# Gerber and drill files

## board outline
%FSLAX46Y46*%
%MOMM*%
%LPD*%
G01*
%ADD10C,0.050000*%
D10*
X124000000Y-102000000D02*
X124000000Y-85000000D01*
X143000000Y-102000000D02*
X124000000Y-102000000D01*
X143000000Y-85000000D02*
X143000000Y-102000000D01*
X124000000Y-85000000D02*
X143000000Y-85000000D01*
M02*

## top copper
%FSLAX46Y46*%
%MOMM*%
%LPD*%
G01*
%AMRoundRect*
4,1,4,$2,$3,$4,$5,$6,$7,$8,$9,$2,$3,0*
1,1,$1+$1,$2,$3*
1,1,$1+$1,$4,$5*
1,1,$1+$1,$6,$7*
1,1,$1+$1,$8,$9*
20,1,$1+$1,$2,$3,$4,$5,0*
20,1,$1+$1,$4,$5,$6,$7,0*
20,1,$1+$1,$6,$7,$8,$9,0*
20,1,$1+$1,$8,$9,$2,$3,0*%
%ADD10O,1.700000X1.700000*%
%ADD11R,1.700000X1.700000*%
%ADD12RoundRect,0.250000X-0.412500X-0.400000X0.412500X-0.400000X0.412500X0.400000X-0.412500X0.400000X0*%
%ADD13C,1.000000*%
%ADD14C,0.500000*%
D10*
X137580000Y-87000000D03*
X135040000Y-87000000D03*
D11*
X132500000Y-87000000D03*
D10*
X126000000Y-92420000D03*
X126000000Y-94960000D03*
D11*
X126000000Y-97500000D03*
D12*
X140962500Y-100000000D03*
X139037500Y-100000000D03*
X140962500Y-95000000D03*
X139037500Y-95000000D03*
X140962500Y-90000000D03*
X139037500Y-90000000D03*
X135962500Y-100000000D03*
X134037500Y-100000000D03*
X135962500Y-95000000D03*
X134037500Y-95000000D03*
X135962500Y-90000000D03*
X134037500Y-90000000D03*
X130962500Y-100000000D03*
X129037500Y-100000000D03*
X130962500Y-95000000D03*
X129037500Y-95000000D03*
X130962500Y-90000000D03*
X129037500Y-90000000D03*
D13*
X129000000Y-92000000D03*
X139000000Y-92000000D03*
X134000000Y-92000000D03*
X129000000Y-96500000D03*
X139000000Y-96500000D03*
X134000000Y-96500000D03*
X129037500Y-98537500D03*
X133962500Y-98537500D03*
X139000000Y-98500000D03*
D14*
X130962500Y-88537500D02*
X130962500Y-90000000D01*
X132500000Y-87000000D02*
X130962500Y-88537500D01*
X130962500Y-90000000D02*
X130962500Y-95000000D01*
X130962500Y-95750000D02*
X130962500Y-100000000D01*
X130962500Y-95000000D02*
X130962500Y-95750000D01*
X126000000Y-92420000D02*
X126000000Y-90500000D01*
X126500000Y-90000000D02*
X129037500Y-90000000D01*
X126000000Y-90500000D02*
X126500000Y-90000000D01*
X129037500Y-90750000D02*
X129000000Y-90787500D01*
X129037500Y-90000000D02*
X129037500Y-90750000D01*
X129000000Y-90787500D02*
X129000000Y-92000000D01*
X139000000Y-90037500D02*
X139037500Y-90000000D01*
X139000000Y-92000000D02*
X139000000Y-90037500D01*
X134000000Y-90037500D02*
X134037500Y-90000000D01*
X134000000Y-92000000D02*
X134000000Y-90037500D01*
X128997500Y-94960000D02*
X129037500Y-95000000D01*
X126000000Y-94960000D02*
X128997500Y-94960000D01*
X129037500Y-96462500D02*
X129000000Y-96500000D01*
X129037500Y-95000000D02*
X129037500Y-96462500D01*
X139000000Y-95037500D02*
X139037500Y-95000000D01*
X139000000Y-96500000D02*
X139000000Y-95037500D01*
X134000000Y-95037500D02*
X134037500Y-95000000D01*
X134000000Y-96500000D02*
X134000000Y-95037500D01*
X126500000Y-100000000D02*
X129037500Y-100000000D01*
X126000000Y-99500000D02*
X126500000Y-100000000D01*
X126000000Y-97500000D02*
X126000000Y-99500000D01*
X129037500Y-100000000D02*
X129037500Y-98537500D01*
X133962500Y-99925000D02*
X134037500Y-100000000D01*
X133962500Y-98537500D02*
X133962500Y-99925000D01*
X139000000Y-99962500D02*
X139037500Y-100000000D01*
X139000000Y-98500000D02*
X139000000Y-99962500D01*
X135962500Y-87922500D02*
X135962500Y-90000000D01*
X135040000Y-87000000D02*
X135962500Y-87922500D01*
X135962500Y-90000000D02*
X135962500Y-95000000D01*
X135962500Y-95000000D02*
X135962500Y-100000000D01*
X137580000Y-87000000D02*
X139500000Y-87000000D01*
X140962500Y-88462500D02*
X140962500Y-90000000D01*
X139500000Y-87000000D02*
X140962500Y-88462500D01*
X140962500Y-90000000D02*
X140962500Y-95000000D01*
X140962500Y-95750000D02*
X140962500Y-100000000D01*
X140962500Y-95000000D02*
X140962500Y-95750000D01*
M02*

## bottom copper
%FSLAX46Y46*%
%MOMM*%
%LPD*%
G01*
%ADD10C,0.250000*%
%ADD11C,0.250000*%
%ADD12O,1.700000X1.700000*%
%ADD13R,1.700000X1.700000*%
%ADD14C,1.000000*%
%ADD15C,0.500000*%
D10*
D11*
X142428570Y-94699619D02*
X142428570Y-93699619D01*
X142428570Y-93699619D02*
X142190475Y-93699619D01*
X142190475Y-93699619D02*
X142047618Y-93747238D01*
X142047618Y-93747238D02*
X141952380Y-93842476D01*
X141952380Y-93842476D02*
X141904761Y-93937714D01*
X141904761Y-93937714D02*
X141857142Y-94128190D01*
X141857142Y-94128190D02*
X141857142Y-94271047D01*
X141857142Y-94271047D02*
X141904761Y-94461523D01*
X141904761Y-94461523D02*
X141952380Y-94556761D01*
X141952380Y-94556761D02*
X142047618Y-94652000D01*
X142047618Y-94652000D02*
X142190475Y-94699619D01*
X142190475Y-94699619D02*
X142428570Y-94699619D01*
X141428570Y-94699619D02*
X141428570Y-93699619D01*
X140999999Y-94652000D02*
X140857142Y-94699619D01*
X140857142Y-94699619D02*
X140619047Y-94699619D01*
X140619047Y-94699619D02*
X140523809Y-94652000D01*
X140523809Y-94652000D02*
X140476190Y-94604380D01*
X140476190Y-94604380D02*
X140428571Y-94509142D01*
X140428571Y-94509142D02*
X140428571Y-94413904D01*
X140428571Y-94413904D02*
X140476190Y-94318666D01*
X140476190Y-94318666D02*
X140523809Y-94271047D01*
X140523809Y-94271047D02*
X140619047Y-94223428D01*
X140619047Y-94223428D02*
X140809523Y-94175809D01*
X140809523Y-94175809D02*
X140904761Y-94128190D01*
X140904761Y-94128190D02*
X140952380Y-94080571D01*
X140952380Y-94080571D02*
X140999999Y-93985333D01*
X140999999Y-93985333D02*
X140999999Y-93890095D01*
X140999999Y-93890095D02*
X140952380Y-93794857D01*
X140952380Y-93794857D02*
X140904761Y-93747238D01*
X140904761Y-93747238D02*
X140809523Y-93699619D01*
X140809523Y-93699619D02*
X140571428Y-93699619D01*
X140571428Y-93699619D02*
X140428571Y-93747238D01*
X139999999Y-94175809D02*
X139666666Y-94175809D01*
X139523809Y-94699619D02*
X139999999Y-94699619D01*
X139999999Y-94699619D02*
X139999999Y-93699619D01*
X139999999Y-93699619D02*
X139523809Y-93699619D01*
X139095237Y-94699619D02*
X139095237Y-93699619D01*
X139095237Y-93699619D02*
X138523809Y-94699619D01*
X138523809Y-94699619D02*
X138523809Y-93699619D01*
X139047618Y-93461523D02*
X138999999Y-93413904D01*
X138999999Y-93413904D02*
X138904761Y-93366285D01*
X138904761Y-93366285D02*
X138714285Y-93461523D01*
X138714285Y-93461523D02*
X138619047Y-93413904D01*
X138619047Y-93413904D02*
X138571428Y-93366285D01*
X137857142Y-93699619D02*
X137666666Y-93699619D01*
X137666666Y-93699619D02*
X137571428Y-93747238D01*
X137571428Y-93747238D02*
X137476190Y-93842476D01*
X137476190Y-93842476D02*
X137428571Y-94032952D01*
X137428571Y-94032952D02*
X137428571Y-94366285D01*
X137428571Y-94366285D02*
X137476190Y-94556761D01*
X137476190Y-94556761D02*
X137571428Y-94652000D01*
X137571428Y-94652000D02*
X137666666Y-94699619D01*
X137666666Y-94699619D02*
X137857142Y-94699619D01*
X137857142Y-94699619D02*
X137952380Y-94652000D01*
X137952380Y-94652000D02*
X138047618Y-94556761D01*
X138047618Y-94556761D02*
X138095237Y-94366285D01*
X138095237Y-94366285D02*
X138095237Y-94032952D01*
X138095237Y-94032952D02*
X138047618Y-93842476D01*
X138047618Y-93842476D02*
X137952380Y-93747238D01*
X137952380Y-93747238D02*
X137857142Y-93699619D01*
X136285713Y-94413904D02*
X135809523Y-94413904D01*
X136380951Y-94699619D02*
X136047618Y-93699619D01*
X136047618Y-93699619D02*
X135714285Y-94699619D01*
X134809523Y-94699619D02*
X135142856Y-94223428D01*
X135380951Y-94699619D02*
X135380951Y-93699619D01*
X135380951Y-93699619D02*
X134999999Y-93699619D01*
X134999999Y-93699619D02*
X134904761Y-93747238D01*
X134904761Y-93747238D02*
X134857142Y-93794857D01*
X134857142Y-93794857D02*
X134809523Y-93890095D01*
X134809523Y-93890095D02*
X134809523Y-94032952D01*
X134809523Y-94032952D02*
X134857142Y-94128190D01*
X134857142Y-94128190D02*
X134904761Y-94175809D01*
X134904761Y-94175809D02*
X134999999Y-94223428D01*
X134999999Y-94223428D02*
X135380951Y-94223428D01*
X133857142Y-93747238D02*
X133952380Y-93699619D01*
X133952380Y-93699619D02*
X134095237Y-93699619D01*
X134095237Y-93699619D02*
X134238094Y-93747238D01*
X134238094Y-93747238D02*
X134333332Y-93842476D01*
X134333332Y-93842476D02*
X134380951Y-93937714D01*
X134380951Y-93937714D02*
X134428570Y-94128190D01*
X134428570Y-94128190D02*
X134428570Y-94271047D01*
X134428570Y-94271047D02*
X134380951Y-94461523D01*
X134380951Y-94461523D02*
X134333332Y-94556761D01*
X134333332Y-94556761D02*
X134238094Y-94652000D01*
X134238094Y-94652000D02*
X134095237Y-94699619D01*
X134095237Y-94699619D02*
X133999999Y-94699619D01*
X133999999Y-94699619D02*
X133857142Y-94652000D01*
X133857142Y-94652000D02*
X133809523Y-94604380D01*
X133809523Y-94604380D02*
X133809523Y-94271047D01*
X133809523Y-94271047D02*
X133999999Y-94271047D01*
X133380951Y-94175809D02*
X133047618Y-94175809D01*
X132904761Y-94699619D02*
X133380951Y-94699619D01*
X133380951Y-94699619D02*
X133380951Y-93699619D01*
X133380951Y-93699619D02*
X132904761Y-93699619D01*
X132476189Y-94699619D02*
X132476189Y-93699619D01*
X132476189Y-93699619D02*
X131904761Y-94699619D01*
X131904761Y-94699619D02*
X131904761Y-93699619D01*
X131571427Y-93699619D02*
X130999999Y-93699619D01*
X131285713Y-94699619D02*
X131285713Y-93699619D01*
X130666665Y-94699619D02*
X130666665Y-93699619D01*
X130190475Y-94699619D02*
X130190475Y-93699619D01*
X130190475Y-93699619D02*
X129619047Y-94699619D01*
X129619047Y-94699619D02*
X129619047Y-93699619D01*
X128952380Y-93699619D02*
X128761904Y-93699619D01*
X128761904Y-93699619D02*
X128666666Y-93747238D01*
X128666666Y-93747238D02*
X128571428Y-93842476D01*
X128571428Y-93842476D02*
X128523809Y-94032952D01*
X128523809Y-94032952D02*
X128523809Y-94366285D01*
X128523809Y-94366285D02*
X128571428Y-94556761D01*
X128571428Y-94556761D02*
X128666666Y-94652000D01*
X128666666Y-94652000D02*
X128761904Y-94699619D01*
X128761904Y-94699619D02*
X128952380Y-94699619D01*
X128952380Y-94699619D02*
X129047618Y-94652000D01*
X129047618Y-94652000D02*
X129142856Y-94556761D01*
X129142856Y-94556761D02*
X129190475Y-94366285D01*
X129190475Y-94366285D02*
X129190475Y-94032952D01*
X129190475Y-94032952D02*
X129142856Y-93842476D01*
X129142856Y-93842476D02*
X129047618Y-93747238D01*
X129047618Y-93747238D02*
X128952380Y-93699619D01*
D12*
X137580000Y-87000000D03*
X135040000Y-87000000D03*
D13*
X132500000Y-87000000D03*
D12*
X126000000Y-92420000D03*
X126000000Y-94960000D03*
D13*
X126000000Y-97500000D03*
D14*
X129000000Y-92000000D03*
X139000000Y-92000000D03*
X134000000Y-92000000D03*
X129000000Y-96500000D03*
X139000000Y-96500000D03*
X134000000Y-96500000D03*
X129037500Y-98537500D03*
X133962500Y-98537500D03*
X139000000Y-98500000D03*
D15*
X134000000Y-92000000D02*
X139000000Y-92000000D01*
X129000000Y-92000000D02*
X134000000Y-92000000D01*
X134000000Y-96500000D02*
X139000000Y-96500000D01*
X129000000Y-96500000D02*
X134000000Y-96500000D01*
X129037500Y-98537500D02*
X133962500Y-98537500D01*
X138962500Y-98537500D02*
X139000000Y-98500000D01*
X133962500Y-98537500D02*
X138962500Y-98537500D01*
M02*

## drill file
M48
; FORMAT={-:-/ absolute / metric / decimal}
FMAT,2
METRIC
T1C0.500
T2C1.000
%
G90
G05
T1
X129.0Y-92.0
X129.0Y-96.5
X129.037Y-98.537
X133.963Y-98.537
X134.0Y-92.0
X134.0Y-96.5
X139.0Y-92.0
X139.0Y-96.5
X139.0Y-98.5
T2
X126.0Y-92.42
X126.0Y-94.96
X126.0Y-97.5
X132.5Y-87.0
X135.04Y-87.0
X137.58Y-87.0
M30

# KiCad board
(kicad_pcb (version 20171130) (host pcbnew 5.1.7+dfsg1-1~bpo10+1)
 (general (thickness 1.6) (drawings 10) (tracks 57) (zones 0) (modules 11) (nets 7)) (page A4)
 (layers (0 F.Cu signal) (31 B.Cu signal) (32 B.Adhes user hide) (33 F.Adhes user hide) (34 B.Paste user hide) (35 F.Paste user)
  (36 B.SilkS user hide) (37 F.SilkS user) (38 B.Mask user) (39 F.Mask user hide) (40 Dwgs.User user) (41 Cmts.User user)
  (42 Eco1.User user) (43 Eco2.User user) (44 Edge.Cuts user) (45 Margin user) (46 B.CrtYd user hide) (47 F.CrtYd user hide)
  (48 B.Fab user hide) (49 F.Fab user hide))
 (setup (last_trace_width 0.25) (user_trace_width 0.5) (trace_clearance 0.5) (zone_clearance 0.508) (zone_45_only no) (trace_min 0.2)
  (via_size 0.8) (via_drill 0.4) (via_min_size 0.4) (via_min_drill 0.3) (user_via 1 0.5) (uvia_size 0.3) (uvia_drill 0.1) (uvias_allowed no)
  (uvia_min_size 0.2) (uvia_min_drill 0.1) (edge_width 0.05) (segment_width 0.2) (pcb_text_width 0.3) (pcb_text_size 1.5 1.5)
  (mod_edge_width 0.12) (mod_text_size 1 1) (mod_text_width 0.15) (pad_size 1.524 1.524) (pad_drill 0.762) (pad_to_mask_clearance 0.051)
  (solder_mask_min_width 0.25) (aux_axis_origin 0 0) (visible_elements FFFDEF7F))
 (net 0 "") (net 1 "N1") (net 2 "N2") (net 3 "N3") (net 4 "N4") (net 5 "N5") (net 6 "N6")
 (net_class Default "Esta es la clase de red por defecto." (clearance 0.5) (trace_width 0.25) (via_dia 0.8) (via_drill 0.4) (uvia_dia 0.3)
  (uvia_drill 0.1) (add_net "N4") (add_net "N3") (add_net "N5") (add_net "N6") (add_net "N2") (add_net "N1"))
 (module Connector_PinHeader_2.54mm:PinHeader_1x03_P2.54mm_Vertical (layer B.Cu) (at 132.5 87 270)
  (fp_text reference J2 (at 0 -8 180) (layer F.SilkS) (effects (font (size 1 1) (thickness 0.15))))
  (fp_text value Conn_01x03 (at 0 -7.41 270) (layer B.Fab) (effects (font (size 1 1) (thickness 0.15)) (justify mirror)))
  (pad 3 thru_hole oval (at 0 -5.08 270) (size 1.7 1.7) (drill 1) (layers *.Cu *.Mask) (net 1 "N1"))
  (pad 2 thru_hole oval (at 0 -2.54 270) (size 1.7 1.7) (drill 1) (layers *.Cu *.Mask) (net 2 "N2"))
  (pad 1 thru_hole rect (at 0 0 270) (size 1.7 1.7) (drill 1) (layers *.Cu *.Mask) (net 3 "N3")))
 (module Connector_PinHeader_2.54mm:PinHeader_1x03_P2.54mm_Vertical (layer B.Cu) (at 126 97.5)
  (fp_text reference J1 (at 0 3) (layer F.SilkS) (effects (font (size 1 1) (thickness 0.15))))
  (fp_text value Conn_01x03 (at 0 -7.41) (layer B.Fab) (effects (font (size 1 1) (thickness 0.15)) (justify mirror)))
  (pad 3 thru_hole oval (at 0 -5.08) (size 1.7 1.7) (drill 1) (layers *.Cu *.Mask) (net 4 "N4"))
  (pad 2 thru_hole oval (at 0 -2.54) (size 1.7 1.7) (drill 1) (layers *.Cu *.Mask) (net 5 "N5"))
  (pad 1 thru_hole rect (at 0 0) (size 1.7 1.7) (drill 1) (layers *.Cu *.Mask) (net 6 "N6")))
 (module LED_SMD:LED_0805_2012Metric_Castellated (layer F.Cu) (at 140 100)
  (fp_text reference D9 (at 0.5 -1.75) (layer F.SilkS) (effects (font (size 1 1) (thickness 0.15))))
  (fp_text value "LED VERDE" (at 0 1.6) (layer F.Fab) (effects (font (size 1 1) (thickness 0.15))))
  (pad 2 smd roundrect (at 0.9625 0) (size 1.325 1.3) (layers F.Cu F.Paste F.Mask) (roundrect_rratio 0.192308) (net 1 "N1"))
  (pad 1 smd roundrect (at -0.9625 0) (size 1.325 1.3) (layers F.Cu F.Paste F.Mask) (roundrect_rratio 0.192308) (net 6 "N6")))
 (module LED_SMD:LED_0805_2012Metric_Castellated (layer F.Cu) (at 140 95)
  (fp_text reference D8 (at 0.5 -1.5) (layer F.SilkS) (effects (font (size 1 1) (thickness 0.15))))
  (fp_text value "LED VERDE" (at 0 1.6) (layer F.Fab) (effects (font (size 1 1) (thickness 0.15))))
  (pad 2 smd roundrect (at 0.9625 0) (size 1.325 1.3) (layers F.Cu F.Paste F.Mask) (roundrect_rratio 0.192308) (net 1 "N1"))
  (pad 1 smd roundrect (at -0.9625 0) (size 1.325 1.3) (layers F.Cu F.Paste F.Mask) (roundrect_rratio 0.192308) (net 5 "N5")))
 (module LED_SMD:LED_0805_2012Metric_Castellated (layer F.Cu) (at 140 90)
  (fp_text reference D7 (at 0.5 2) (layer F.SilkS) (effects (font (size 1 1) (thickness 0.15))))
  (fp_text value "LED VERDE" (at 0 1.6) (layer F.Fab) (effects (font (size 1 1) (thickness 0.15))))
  (pad 2 smd roundrect (at 0.9625 0) (size 1.325 1.3) (layers F.Cu F.Paste F.Mask) (roundrect_rratio 0.192308) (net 1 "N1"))
  (pad 1 smd roundrect (at -0.9625 0) (size 1.325 1.3) (layers F.Cu F.Paste F.Mask) (roundrect_rratio 0.192308) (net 4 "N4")))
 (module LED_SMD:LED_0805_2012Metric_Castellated (layer F.Cu) (at 135 100)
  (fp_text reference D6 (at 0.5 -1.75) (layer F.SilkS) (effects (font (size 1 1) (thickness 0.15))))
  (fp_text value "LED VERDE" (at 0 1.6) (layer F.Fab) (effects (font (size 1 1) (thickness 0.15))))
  (pad 2 smd roundrect (at 0.9625 0) (size 1.325 1.3) (layers F.Cu F.Paste F.Mask) (roundrect_rratio 0.192308) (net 2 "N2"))
  (pad 1 smd roundrect (at -0.9625 0) (size 1.325 1.3) (layers F.Cu F.Paste F.Mask) (roundrect_rratio 0.192308) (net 6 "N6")))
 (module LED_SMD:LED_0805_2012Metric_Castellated (layer F.Cu) (at 135 95)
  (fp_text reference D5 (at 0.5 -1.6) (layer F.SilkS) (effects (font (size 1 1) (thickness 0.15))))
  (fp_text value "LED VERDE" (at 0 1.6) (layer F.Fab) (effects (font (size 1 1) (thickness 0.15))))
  (pad 2 smd roundrect (at 0.9625 0) (size 1.325 1.3) (layers F.Cu F.Paste F.Mask) (roundrect_rratio 0.192308) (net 2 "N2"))
  (pad 1 smd roundrect (at -0.9625 0) (size 1.325 1.3) (layers F.Cu F.Paste F.Mask) (roundrect_rratio 0.192308) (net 5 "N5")))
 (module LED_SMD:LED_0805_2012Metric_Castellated (layer F.Cu) (at 135 90)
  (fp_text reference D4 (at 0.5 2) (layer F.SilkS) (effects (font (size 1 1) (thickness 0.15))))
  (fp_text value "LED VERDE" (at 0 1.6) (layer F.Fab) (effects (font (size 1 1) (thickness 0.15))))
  (pad 2 smd roundrect (at 0.9625 0) (size 1.325 1.3) (layers F.Cu F.Paste F.Mask) (roundrect_rratio 0.192308) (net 2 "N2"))
  (pad 1 smd roundrect (at -0.9625 0) (size 1.325 1.3) (layers F.Cu F.Paste F.Mask) (roundrect_rratio 0.192308) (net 4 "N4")))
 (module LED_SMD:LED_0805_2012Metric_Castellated (layer F.Cu) (at 130 100)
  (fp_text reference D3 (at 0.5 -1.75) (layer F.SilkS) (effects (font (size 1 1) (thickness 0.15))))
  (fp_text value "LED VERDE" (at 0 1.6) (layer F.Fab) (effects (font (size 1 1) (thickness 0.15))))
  (pad 2 smd roundrect (at 0.9625 0) (size 1.325 1.3) (layers F.Cu F.Paste F.Mask) (roundrect_rratio 0.192308) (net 3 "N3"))
  (pad 1 smd roundrect (at -0.9625 0) (size 1.325 1.3) (layers F.Cu F.Paste F.Mask) (roundrect_rratio 0.192308) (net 6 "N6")))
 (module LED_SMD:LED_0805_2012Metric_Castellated (layer F.Cu) (at 130 95)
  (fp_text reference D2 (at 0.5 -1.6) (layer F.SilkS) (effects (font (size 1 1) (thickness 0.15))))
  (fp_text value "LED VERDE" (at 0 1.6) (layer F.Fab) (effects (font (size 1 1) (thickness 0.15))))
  (pad 2 smd roundrect (at 0.9625 0) (size 1.325 1.3) (layers F.Cu F.Paste F.Mask) (roundrect_rratio 0.192308) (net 3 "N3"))
  (pad 1 smd roundrect (at -0.9625 0) (size 1.325 1.3) (layers F.Cu F.Paste F.Mask) (roundrect_rratio 0.192308) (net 5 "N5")))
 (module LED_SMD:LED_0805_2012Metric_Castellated (layer F.Cu) (at 130 90)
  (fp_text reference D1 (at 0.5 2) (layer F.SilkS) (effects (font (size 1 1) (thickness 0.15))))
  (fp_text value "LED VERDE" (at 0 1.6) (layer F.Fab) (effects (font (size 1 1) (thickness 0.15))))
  (pad 2 smd roundrect (at 0.9625 0) (size 1.325 1.3) (layers F.Cu F.Paste F.Mask) (roundrect_rratio 0.192308) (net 3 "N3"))
  (pad 1 smd roundrect (at -0.9625 0) (size 1.325 1.3) (layers F.Cu F.Paste F.Mask) (roundrect_rratio 0.192308) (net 4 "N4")))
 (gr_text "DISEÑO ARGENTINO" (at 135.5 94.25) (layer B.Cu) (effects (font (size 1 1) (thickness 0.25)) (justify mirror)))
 (gr_line (start 124 102) (end 124 85) (layer Edge.Cuts) (width 0.05))
 (gr_line (start 143 102) (end 124 102) (layer Edge.Cuts) (width 0.05))
 (gr_line (start 143 85) (end 143 102) (layer Edge.Cuts) (width 0.05))
 (gr_line (start 124 85) (end 143 85) (layer Edge.Cuts) (width 0.05))
 (segment (start 130.9625 88.5375) (end 130.9625 90) (width 0.5) (layer F.Cu) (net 3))
 (segment (start 132.5 87) (end 130.9625 88.5375) (width 0.5) (layer F.Cu) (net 3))
 (segment (start 130.9625 90) (end 130.9625 95) (width 0.5) (layer F.Cu) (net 3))
 (segment (start 130.9625 95.75) (end 130.9625 100) (width 0.5) (layer F.Cu) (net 3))
 (segment (start 130.9625 95) (end 130.9625 95.75) (width 0.5) (layer F.Cu) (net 3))
 (segment (start 126 92.42) (end 126 90.5) (width 0.5) (layer F.Cu) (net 4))
 (segment (start 126.5 90) (end 129.0375 90) (width 0.5) (layer F.Cu) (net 4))
 (segment (start 126 90.5) (end 126.5 90) (width 0.5) (layer F.Cu) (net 4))
 (segment (start 129.0375 90.75) (end 129 90.7875) (width 0.5) (layer F.Cu) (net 4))
 (segment (start 129.0375 90) (end 129.0375 90.75) (width 0.5) (layer F.Cu) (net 4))
 (via (at 129 92) (size 1) (drill 0.5) (layers F.Cu B.Cu) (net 4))
 (segment (start 129 90.7875) (end 129 92) (width 0.5) (layer F.Cu) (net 4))
 (via (at 139 92) (size 1) (drill 0.5) (layers F.Cu B.Cu) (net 4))
 (segment (start 139 90.0375) (end 139.0375 90) (width 0.5) (layer F.Cu) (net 4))
 (segment (start 139 92) (end 139 90.0375) (width 0.5) (layer F.Cu) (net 4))
 (segment (start 134 92) (end 139 92) (width 0.5) (layer B.Cu) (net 4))
 (segment (start 129 92) (end 134 92) (width 0.5) (layer B.Cu) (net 4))
 (via (at 134 92) (size 1) (drill 0.5) (layers F.Cu B.Cu) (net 4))
 (segment (start 134 90.0375) (end 134.0375 90) (width 0.5) (layer F.Cu) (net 4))
 (segment (start 134 92) (end 134 90.0375) (width 0.5) (layer F.Cu) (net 4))
 (segment (start 128.9975 94.96) (end 129.0375 95) (width 0.5) (layer F.Cu) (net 5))
 (segment (start 126 94.96) (end 128.9975 94.96) (width 0.5) (layer F.Cu) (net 5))
 (via (at 129 96.5) (size 1) (drill 0.5) (layers F.Cu B.Cu) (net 5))
 (segment (start 129.0375 96.4625) (end 129 96.5) (width 0.5) (layer F.Cu) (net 5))
 (segment (start 129.0375 95) (end 129.0375 96.4625) (width 0.5) (layer F.Cu) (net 5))
 (via (at 139 96.5) (size 1) (drill 0.5) (layers F.Cu B.Cu) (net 5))
 (segment (start 139 95.0375) (end 139.0375 95) (width 0.5) (layer F.Cu) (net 5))
 (segment (start 139 96.5) (end 139 95.0375) (width 0.5) (layer F.Cu) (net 5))
 (segment (start 134 96.5) (end 139 96.5) (width 0.5) (layer B.Cu) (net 5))
 (segment (start 129 96.5) (end 134 96.5) (width 0.5) (layer B.Cu) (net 5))
 (via (at 134 96.5) (size 1) (drill 0.5) (layers F.Cu B.Cu) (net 5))
 (segment (start 134 95.0375) (end 134.0375 95) (width 0.5) (layer F.Cu) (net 5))
 (segment (start 134 96.5) (end 134 95.0375) (width 0.5) (layer F.Cu) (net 5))
 (segment (start 126.5 100) (end 129.0375 100) (width 0.5) (layer F.Cu) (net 6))
 (segment (start 126 99.5) (end 126.5 100) (width 0.5) (layer F.Cu) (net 6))
 (segment (start 126 97.5) (end 126 99.5) (width 0.5) (layer F.Cu) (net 6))
 (segment (start 129.0375 100) (end 129.0375 98.5375) (width 0.5) (layer F.Cu) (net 6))
 (via (at 129.0375 98.5375) (size 1) (drill 0.5) (layers F.Cu B.Cu) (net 6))
 (segment (start 129.0375 98.5375) (end 133.9625 98.5375) (width 0.5) (layer B.Cu) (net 6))
 (via (at 133.9625 98.5375) (size 1) (drill 0.5) (layers F.Cu B.Cu) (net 6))
 (segment (start 133.9625 99.925) (end 134.0375 100) (width 0.5) (layer F.Cu) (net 6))
 (segment (start 133.9625 98.5375) (end 133.9625 99.925) (width 0.5) (layer F.Cu) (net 6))
 (segment (start 138.9625 98.5375) (end 139 98.5) (width 0.5) (layer B.Cu) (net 6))
 (via (at 139 98.5) (size 1) (drill 0.5) (layers F.Cu B.Cu) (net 6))
 (segment (start 133.9625 98.5375) (end 138.9625 98.5375) (width 0.5) (layer B.Cu) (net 6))
 (segment (start 139 99.9625) (end 139.0375 100) (width 0.5) (layer F.Cu) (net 6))
 (segment (start 139 98.5) (end 139 99.9625) (width 0.5) (layer F.Cu) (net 6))
 (segment (start 135.9625 87.9225) (end 135.9625 90) (width 0.5) (layer F.Cu) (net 2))
 (segment (start 135.04 87) (end 135.9625 87.9225) (width 0.5) (layer F.Cu) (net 2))
 (segment (start 135.9625 90) (end 135.9625 95) (width 0.5) (layer F.Cu) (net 2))
 (segment (start 135.9625 95) (end 135.9625 100) (width 0.5) (layer F.Cu) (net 2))
 (segment (start 137.58 87) (end 139.5 87) (width 0.5) (layer F.Cu) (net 1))
 (segment (start 140.9625 88.4625) (end 140.9625 90) (width 0.5) (layer F.Cu) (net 1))
 (segment (start 139.5 87) (end 140.9625 88.4625) (width 0.5) (layer F.Cu) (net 1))
 (segment (start 140.9625 90) (end 140.9625 95) (width 0.5) (layer F.Cu) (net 1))
 (segment (start 140.9625 95.75) (end 140.9625 100) (width 0.5) (layer F.Cu) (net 1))
 (segment (start 140.9625 95) (end 140.9625 95.75) (width 0.5) (layer F.Cu) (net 1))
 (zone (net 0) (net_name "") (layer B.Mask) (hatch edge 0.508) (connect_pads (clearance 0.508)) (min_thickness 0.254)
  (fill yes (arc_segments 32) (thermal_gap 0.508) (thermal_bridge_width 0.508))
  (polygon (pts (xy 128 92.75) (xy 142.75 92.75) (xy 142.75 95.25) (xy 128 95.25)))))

